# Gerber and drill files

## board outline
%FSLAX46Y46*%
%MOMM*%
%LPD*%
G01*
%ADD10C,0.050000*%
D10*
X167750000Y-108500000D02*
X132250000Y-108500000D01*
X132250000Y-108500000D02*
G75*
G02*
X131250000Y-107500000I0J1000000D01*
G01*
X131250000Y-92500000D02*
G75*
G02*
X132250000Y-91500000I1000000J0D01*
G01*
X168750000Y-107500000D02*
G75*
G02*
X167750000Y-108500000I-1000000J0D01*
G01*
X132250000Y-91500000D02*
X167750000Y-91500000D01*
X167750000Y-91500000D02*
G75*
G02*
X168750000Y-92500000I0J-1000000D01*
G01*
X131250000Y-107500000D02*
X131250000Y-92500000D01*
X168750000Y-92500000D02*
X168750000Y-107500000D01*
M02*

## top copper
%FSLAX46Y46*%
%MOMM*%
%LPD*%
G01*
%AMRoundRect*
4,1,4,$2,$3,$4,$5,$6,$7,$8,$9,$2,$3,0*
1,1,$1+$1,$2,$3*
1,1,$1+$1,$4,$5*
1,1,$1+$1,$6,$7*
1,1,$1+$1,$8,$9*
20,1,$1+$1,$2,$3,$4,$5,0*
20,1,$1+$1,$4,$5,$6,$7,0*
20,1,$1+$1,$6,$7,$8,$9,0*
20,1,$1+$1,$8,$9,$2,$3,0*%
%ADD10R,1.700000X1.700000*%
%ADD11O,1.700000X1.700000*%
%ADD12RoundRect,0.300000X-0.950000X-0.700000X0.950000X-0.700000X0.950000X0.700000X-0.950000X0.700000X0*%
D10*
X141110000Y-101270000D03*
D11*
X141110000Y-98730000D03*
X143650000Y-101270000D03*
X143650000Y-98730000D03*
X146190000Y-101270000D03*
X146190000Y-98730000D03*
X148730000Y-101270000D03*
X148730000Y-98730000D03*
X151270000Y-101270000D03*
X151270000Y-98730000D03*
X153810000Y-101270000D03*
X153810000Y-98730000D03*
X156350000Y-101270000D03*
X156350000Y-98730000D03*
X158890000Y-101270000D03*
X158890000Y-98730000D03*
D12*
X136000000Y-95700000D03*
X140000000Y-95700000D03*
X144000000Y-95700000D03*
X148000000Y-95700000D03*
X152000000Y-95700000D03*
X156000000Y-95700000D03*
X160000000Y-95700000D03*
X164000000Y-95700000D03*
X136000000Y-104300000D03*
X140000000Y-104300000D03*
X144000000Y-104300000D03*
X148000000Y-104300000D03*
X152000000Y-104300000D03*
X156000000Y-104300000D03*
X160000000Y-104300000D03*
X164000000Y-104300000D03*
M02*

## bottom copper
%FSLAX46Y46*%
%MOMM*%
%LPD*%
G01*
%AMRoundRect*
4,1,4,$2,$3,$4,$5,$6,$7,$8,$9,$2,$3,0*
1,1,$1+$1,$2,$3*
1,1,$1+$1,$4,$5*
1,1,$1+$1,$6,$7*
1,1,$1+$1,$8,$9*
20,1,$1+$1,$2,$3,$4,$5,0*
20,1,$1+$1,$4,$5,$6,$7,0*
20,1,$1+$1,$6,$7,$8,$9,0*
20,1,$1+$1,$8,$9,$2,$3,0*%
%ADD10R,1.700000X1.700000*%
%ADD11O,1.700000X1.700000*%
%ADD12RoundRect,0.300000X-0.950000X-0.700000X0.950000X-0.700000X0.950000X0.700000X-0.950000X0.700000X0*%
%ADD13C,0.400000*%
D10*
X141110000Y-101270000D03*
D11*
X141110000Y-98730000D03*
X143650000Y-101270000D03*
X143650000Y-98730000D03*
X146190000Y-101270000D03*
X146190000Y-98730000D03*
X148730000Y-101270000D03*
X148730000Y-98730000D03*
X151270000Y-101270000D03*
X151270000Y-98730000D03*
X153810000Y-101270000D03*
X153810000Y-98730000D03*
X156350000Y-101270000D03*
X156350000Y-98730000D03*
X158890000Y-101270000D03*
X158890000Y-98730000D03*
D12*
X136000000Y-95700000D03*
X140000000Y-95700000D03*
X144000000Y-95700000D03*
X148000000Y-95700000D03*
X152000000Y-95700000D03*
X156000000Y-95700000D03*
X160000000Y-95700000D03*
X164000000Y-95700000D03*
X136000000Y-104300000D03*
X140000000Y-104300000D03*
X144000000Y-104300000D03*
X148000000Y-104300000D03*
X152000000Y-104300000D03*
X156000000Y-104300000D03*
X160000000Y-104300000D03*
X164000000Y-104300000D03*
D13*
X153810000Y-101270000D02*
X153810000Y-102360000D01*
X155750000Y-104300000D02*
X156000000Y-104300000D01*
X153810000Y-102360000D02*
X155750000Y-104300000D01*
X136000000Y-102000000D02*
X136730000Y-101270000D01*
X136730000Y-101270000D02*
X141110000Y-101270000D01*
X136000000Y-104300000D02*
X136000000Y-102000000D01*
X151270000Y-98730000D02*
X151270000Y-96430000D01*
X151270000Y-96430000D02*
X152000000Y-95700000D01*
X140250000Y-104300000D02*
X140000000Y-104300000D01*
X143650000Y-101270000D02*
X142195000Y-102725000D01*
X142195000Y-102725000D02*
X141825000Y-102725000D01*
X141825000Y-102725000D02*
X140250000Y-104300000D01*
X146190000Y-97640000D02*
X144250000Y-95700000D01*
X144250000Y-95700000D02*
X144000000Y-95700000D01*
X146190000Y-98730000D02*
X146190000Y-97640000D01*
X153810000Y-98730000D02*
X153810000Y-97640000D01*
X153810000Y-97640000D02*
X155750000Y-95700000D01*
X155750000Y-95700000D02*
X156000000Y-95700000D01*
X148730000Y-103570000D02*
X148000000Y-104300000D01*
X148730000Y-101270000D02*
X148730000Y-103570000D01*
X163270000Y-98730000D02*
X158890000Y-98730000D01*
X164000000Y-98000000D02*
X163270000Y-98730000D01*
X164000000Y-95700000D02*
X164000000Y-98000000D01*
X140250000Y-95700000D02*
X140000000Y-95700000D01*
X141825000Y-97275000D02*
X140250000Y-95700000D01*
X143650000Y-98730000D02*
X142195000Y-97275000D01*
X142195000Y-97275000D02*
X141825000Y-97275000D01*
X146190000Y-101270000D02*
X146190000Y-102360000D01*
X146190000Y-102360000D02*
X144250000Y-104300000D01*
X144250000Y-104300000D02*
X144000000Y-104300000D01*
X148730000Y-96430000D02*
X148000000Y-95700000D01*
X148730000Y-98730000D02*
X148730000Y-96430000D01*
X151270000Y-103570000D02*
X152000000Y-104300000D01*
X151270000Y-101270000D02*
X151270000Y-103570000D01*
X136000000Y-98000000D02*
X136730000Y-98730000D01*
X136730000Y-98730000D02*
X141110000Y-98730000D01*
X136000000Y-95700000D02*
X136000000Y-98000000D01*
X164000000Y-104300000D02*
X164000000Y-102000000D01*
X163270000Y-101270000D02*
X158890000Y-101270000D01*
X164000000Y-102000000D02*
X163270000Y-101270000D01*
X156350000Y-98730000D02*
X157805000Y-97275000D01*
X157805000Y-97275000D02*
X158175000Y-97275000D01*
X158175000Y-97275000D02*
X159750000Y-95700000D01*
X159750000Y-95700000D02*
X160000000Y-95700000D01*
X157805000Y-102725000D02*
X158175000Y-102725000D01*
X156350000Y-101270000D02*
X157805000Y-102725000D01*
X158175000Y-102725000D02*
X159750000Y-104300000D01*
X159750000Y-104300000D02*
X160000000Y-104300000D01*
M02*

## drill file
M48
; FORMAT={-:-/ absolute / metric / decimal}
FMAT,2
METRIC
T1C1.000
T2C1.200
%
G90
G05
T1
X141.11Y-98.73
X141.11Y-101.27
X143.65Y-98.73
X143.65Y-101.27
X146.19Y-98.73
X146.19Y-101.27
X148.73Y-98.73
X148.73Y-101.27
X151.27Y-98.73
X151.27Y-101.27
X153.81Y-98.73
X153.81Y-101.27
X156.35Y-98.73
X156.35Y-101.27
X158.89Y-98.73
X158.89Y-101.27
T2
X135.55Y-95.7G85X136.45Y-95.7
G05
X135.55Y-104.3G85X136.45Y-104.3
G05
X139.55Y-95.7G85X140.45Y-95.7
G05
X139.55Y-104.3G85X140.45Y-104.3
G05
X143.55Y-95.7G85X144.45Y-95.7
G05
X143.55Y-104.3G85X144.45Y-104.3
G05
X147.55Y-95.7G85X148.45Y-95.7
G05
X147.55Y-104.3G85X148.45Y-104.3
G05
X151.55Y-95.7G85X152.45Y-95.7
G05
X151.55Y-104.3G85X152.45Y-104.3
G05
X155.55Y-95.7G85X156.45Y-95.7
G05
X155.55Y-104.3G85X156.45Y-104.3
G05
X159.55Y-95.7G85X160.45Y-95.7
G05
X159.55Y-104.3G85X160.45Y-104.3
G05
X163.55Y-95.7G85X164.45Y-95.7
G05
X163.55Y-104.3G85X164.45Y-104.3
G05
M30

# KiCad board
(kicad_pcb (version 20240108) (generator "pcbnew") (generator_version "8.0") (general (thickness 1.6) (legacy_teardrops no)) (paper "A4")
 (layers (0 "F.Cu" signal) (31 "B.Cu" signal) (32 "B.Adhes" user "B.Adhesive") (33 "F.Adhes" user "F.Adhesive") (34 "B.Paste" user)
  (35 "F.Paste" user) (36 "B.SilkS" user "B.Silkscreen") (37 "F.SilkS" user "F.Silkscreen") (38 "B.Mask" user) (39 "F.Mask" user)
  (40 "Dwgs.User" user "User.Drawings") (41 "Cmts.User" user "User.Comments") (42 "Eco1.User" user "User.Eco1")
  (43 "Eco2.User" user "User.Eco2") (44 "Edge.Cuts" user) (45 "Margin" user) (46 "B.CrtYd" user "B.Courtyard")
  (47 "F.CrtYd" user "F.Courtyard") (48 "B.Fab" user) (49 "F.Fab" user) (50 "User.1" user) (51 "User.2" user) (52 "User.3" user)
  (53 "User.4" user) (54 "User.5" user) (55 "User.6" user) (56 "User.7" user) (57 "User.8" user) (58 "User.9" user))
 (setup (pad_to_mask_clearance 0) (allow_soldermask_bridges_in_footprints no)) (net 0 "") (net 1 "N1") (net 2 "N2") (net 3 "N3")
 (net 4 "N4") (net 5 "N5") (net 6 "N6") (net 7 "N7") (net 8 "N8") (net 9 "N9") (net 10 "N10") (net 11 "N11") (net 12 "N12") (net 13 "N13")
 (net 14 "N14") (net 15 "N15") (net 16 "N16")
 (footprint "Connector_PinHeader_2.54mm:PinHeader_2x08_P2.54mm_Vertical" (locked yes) (layer "F.Cu") (at 141.11 101.27 90)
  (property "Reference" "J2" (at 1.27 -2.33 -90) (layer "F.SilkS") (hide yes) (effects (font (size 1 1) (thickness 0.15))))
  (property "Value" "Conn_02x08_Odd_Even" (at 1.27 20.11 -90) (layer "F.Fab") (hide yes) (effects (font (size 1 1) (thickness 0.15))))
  (pad "1" thru_hole rect (at 0 0 90) (size 1.7 1.7) (drill 1) (layers "*.Cu" "*.Mask") (remove_unused_layers no) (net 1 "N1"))
  (pad "2" thru_hole oval (at 2.54 0 90) (size 1.7 1.7) (drill 1) (layers "*.Cu" "*.Mask") (remove_unused_layers no) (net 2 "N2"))
  (pad "3" thru_hole oval (at 0 2.54 90) (size 1.7 1.7) (drill 1) (layers "*.Cu" "*.Mask") (remove_unused_layers no) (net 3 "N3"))
  (pad "4" thru_hole oval (at 2.54 2.54 90) (size 1.7 1.7) (drill 1) (layers "*.Cu" "*.Mask") (remove_unused_layers no) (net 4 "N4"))
  (pad "5" thru_hole oval (at 0 5.08 90) (size 1.7 1.7) (drill 1) (layers "*.Cu" "*.Mask") (remove_unused_layers no) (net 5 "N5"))
  (pad "6" thru_hole oval (at 2.54 5.08 90) (size 1.7 1.7) (drill 1) (layers "*.Cu" "*.Mask") (remove_unused_layers no) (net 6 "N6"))
  (pad "7" thru_hole oval (at 0 7.62 90) (size 1.7 1.7) (drill 1) (layers "*.Cu" "*.Mask") (remove_unused_layers no) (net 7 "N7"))
  (pad "8" thru_hole oval (at 2.54 7.62 90) (size 1.7 1.7) (drill 1) (layers "*.Cu" "*.Mask") (remove_unused_layers no) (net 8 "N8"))
  (pad "9" thru_hole oval (at 0 10.16 90) (size 1.7 1.7) (drill 1) (layers "*.Cu" "*.Mask") (remove_unused_layers no) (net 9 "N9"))
  (pad "10" thru_hole oval (at 2.54 10.16 90) (size 1.7 1.7) (drill 1) (layers "*.Cu" "*.Mask") (remove_unused_layers no) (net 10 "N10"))
  (pad "11" thru_hole oval (at 0 12.7 90) (size 1.7 1.7) (drill 1) (layers "*.Cu" "*.Mask") (remove_unused_layers no) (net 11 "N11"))
  (pad "12" thru_hole oval (at 2.54 12.7 90) (size 1.7 1.7) (drill 1) (layers "*.Cu" "*.Mask") (remove_unused_layers no) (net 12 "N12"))
  (pad "13" thru_hole oval (at 0 15.24 90) (size 1.7 1.7) (drill 1) (layers "*.Cu" "*.Mask") (remove_unused_layers no) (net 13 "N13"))
  (pad "14" thru_hole oval (at 2.54 15.24 90) (size 1.7 1.7) (drill 1) (layers "*.Cu" "*.Mask") (remove_unused_layers no) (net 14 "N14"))
  (pad "15" thru_hole oval (at 0 17.78 90) (size 1.7 1.7) (drill 1) (layers "*.Cu" "*.Mask") (remove_unused_layers no) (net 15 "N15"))
  (pad "16" thru_hole oval (at 2.54 17.78 90) (size 1.7 1.7) (drill 1) (layers "*.Cu" "*.Mask") (remove_unused_layers no) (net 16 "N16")))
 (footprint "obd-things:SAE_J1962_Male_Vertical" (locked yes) (layer "B.Cu") (at 150 100 -90)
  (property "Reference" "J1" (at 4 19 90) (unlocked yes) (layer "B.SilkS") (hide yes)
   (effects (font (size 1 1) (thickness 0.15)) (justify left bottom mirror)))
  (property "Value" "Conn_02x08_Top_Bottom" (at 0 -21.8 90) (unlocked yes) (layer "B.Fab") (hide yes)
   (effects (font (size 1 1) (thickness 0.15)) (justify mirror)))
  (pad "1" thru_hole roundrect (at -4.3 14) (size 2.5 2) (drill oval 2.1 1.2) (layers "*.Cu" "*.Mask") (remove_unused_layers no)
   (roundrect_rratio 0.15) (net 2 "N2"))
  (pad "2" thru_hole roundrect (at -4.3 10) (size 2.5 2) (drill oval 2.1 1.2) (layers "*.Cu" "*.Mask") (remove_unused_layers no)
   (roundrect_rratio 0.15) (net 4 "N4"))
  (pad "3" thru_hole roundrect (at -4.3 6) (size 2.5 2) (drill oval 2.1 1.2) (layers "*.Cu" "*.Mask") (remove_unused_layers no)
   (roundrect_rratio 0.15) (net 6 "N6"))
  (pad "4" thru_hole roundrect (at -4.3 2) (size 2.5 2) (drill oval 2.1 1.2) (layers "*.Cu" "*.Mask") (remove_unused_layers no)
   (roundrect_rratio 0.15) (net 8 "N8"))
  (pad "5" thru_hole roundrect (at -4.3 -2) (size 2.5 2) (drill oval 2.1 1.2) (layers "*.Cu" "*.Mask") (remove_unused_layers no)
   (roundrect_rratio 0.15) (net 10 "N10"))
  (pad "6" thru_hole roundrect (at -4.3 -6) (size 2.5 2) (drill oval 2.1 1.2) (layers "*.Cu" "*.Mask") (remove_unused_layers no)
   (roundrect_rratio 0.15) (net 12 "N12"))
  (pad "7" thru_hole roundrect (at -4.3 -10) (size 2.5 2) (drill oval 2.1 1.2) (layers "*.Cu" "*.Mask") (remove_unused_layers no)
   (roundrect_rratio 0.15) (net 14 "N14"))
  (pad "8" thru_hole roundrect (at -4.3 -14) (size 2.5 2) (drill oval 2.1 1.2) (layers "*.Cu" "*.Mask") (remove_unused_layers no)
   (roundrect_rratio 0.15) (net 16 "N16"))
  (pad "9" thru_hole roundrect (at 4.3 14) (size 2.5 2) (drill oval 2.1 1.2) (layers "*.Cu" "*.Mask") (remove_unused_layers no)
   (roundrect_rratio 0.15) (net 1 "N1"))
  (pad "10" thru_hole roundrect (at 4.3 10) (size 2.5 2) (drill oval 2.1 1.2) (layers "*.Cu" "*.Mask") (remove_unused_layers no)
   (roundrect_rratio 0.15) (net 3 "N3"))
  (pad "11" thru_hole roundrect (at 4.3 6) (size 2.5 2) (drill oval 2.1 1.2) (layers "*.Cu" "*.Mask") (remove_unused_layers no)
   (roundrect_rratio 0.15) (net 5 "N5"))
  (pad "12" thru_hole roundrect (at 4.3 2) (size 2.5 2) (drill oval 2.1 1.2) (layers "*.Cu" "*.Mask") (remove_unused_layers no)
   (roundrect_rratio 0.15) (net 7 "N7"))
  (pad "13" thru_hole roundrect (at 4.3 -2) (size 2.5 2) (drill oval 2.1 1.2) (layers "*.Cu" "*.Mask") (remove_unused_layers no)
   (roundrect_rratio 0.15) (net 9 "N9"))
  (pad "14" thru_hole roundrect (at 4.3 -6) (size 2.5 2) (drill oval 2.1 1.2) (layers "*.Cu" "*.Mask") (remove_unused_layers no)
   (roundrect_rratio 0.15) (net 11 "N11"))
  (pad "15" thru_hole roundrect (at 4.3 -10) (size 2.5 2) (drill oval 2.1 1.2) (layers "*.Cu" "*.Mask") (remove_unused_layers no)
   (roundrect_rratio 0.15) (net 13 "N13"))
  (pad "16" thru_hole roundrect (at 4.3 -14) (size 2.5 2) (drill oval 2.1 1.2) (layers "*.Cu" "*.Mask") (remove_unused_layers no)
   (roundrect_rratio 0.15) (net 15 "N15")))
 (gr_line (start 167.75 108.5) (end 132.25 108.5) (locked yes) (stroke (width 0.05) (type default)) (layer "Edge.Cuts"))
 (gr_arc (start 132.25 108.5) (mid 131.542893 108.207107) (end 131.25 107.5) (locked yes) (stroke (width 0.05) (type default))
  (layer "Edge.Cuts"))
 (gr_arc (start 131.25 92.5) (mid 131.542893 91.792893) (end 132.25 91.5) (locked yes) (stroke (width 0.05) (type default))
  (layer "Edge.Cuts"))
 (gr_arc (start 168.75 107.5) (mid 168.457107 108.207107) (end 167.75 108.5) (locked yes) (stroke (width 0.05) (type default))
  (layer "Edge.Cuts"))
 (gr_line (start 132.25 91.5) (end 167.75 91.5) (locked yes) (stroke (width 0.05) (type default)) (layer "Edge.Cuts"))
 (gr_arc (start 167.75 91.5) (mid 168.457107 91.792893) (end 168.75 92.5) (locked yes) (stroke (width 0.05) (type default))
  (layer "Edge.Cuts"))
 (gr_line (start 131.25 107.5) (end 131.25 92.5) (locked yes) (stroke (width 0.05) (type default)) (layer "Edge.Cuts"))
 (gr_line (start 168.75 92.5) (end 168.75 107.5) (locked yes) (stroke (width 0.05) (type default)) (layer "Edge.Cuts"))
 (segment (start 153.81 101.27) (end 153.81 102.36) (width 0.4) (locked yes) (layer "B.Cu") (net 11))
 (segment (start 155.75 104.3) (end 156 104.3) (width 0.4) (locked yes) (layer "B.Cu") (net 11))
 (segment (start 153.81 102.36) (end 155.75 104.3) (width 0.4) (locked yes) (layer "B.Cu") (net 11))
 (segment (start 136 102) (end 136.73 101.27) (width 0.4) (locked yes) (layer "B.Cu") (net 1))
 (segment (start 136.73 101.27) (end 141.11 101.27) (width 0.4) (locked yes) (layer "B.Cu") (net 1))
 (segment (start 136 104.3) (end 136 102) (width 0.4) (locked yes) (layer "B.Cu") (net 1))
 (segment (start 151.27 98.73) (end 151.27 96.43) (width 0.4) (locked yes) (layer "B.Cu") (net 10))
 (segment (start 151.27 96.43) (end 152 95.7) (width 0.4) (locked yes) (layer "B.Cu") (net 10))
 (segment (start 140.25 104.3) (end 140 104.3) (width 0.4) (locked yes) (layer "B.Cu") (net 3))
 (segment (start 143.65 101.27) (end 142.195 102.725) (width 0.4) (locked yes) (layer "B.Cu") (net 3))
 (segment (start 142.195 102.725) (end 141.825 102.725) (width 0.4) (locked yes) (layer "B.Cu") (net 3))
 (segment (start 141.825 102.725) (end 140.25 104.3) (width 0.4) (locked yes) (layer "B.Cu") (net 3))
 (segment (start 146.19 97.64) (end 144.25 95.7) (width 0.4) (locked yes) (layer "B.Cu") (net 6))
 (segment (start 144.25 95.7) (end 144 95.7) (width 0.4) (locked yes) (layer "B.Cu") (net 6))
 (segment (start 146.19 98.73) (end 146.19 97.64) (width 0.4) (locked yes) (layer "B.Cu") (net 6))
 (segment (start 153.81 98.73) (end 153.81 97.64) (width 0.4) (locked yes) (layer "B.Cu") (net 12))
 (segment (start 153.81 97.64) (end 155.75 95.7) (width 0.4) (locked yes) (layer "B.Cu") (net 12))
 (segment (start 155.75 95.7) (end 156 95.7) (width 0.4) (locked yes) (layer "B.Cu") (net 12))
 (segment (start 148.73 103.57) (end 148 104.3) (width 0.4) (locked yes) (layer "B.Cu") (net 7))
 (segment (start 148.73 101.27) (end 148.73 103.57) (width 0.4) (locked yes) (layer "B.Cu") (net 7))
 (segment (start 163.27 98.73) (end 158.89 98.73) (width 0.4) (locked yes) (layer "B.Cu") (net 16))
 (segment (start 164 98) (end 163.27 98.73) (width 0.4) (locked yes) (layer "B.Cu") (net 16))
 (segment (start 164 95.7) (end 164 98) (width 0.4) (locked yes) (layer "B.Cu") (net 16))
 (segment (start 140.25 95.7) (end 140 95.7) (width 0.4) (locked yes) (layer "B.Cu") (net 4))
 (segment (start 141.825 97.275) (end 140.25 95.7) (width 0.4) (locked yes) (layer "B.Cu") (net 4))
 (segment (start 143.65 98.73) (end 142.195 97.275) (width 0.4) (locked yes) (layer "B.Cu") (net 4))
 (segment (start 142.195 97.275) (end 141.825 97.275) (width 0.4) (locked yes) (layer "B.Cu") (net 4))
 (segment (start 146.19 101.27) (end 146.19 102.36) (width 0.4) (locked yes) (layer "B.Cu") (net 5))
 (segment (start 146.19 102.36) (end 144.25 104.3) (width 0.4) (locked yes) (layer "B.Cu") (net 5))
 (segment (start 144.25 104.3) (end 144 104.3) (width 0.4) (locked yes) (layer "B.Cu") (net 5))
 (segment (start 148.73 96.43) (end 148 95.7) (width 0.4) (locked yes) (layer "B.Cu") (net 8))
 (segment (start 148.73 98.73) (end 148.73 96.43) (width 0.4) (locked yes) (layer "B.Cu") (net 8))
 (segment (start 151.27 103.57) (end 152 104.3) (width 0.4) (locked yes) (layer "B.Cu") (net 9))
 (segment (start 151.27 101.27) (end 151.27 103.57) (width 0.4) (locked yes) (layer "B.Cu") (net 9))
 (segment (start 136 98) (end 136.73 98.73) (width 0.4) (locked yes) (layer "B.Cu") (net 2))
 (segment (start 136.73 98.73) (end 141.11 98.73) (width 0.4) (locked yes) (layer "B.Cu") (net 2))
 (segment (start 136 95.7) (end 136 98) (width 0.4) (locked yes) (layer "B.Cu") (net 2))
 (segment (start 164 104.3) (end 164 102) (width 0.4) (locked yes) (layer "B.Cu") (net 15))
 (segment (start 163.27 101.27) (end 158.89 101.27) (width 0.4) (locked yes) (layer "B.Cu") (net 15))
 (segment (start 164 102) (end 163.27 101.27) (width 0.4) (locked yes) (layer "B.Cu") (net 15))
 (segment (start 156.35 98.73) (end 157.805 97.275) (width 0.4) (locked yes) (layer "B.Cu") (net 14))
 (segment (start 157.805 97.275) (end 158.175 97.275) (width 0.4) (locked yes) (layer "B.Cu") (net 14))
 (segment (start 158.175 97.275) (end 159.75 95.7) (width 0.4) (locked yes) (layer "B.Cu") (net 14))
 (segment (start 159.75 95.7) (end 160 95.7) (width 0.4) (locked yes) (layer "B.Cu") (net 14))
 (segment (start 157.805 102.725) (end 158.175 102.725) (width 0.4) (locked yes) (layer "B.Cu") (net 13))
 (segment (start 156.35 101.27) (end 157.805 102.725) (width 0.4) (locked yes) (layer "B.Cu") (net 13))
 (segment (start 158.175 102.725) (end 159.75 104.3) (width 0.4) (locked yes) (layer "B.Cu") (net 13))
 (segment (start 159.75 104.3) (end 160 104.3) (width 0.4) (locked yes) (layer "B.Cu") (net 13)))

